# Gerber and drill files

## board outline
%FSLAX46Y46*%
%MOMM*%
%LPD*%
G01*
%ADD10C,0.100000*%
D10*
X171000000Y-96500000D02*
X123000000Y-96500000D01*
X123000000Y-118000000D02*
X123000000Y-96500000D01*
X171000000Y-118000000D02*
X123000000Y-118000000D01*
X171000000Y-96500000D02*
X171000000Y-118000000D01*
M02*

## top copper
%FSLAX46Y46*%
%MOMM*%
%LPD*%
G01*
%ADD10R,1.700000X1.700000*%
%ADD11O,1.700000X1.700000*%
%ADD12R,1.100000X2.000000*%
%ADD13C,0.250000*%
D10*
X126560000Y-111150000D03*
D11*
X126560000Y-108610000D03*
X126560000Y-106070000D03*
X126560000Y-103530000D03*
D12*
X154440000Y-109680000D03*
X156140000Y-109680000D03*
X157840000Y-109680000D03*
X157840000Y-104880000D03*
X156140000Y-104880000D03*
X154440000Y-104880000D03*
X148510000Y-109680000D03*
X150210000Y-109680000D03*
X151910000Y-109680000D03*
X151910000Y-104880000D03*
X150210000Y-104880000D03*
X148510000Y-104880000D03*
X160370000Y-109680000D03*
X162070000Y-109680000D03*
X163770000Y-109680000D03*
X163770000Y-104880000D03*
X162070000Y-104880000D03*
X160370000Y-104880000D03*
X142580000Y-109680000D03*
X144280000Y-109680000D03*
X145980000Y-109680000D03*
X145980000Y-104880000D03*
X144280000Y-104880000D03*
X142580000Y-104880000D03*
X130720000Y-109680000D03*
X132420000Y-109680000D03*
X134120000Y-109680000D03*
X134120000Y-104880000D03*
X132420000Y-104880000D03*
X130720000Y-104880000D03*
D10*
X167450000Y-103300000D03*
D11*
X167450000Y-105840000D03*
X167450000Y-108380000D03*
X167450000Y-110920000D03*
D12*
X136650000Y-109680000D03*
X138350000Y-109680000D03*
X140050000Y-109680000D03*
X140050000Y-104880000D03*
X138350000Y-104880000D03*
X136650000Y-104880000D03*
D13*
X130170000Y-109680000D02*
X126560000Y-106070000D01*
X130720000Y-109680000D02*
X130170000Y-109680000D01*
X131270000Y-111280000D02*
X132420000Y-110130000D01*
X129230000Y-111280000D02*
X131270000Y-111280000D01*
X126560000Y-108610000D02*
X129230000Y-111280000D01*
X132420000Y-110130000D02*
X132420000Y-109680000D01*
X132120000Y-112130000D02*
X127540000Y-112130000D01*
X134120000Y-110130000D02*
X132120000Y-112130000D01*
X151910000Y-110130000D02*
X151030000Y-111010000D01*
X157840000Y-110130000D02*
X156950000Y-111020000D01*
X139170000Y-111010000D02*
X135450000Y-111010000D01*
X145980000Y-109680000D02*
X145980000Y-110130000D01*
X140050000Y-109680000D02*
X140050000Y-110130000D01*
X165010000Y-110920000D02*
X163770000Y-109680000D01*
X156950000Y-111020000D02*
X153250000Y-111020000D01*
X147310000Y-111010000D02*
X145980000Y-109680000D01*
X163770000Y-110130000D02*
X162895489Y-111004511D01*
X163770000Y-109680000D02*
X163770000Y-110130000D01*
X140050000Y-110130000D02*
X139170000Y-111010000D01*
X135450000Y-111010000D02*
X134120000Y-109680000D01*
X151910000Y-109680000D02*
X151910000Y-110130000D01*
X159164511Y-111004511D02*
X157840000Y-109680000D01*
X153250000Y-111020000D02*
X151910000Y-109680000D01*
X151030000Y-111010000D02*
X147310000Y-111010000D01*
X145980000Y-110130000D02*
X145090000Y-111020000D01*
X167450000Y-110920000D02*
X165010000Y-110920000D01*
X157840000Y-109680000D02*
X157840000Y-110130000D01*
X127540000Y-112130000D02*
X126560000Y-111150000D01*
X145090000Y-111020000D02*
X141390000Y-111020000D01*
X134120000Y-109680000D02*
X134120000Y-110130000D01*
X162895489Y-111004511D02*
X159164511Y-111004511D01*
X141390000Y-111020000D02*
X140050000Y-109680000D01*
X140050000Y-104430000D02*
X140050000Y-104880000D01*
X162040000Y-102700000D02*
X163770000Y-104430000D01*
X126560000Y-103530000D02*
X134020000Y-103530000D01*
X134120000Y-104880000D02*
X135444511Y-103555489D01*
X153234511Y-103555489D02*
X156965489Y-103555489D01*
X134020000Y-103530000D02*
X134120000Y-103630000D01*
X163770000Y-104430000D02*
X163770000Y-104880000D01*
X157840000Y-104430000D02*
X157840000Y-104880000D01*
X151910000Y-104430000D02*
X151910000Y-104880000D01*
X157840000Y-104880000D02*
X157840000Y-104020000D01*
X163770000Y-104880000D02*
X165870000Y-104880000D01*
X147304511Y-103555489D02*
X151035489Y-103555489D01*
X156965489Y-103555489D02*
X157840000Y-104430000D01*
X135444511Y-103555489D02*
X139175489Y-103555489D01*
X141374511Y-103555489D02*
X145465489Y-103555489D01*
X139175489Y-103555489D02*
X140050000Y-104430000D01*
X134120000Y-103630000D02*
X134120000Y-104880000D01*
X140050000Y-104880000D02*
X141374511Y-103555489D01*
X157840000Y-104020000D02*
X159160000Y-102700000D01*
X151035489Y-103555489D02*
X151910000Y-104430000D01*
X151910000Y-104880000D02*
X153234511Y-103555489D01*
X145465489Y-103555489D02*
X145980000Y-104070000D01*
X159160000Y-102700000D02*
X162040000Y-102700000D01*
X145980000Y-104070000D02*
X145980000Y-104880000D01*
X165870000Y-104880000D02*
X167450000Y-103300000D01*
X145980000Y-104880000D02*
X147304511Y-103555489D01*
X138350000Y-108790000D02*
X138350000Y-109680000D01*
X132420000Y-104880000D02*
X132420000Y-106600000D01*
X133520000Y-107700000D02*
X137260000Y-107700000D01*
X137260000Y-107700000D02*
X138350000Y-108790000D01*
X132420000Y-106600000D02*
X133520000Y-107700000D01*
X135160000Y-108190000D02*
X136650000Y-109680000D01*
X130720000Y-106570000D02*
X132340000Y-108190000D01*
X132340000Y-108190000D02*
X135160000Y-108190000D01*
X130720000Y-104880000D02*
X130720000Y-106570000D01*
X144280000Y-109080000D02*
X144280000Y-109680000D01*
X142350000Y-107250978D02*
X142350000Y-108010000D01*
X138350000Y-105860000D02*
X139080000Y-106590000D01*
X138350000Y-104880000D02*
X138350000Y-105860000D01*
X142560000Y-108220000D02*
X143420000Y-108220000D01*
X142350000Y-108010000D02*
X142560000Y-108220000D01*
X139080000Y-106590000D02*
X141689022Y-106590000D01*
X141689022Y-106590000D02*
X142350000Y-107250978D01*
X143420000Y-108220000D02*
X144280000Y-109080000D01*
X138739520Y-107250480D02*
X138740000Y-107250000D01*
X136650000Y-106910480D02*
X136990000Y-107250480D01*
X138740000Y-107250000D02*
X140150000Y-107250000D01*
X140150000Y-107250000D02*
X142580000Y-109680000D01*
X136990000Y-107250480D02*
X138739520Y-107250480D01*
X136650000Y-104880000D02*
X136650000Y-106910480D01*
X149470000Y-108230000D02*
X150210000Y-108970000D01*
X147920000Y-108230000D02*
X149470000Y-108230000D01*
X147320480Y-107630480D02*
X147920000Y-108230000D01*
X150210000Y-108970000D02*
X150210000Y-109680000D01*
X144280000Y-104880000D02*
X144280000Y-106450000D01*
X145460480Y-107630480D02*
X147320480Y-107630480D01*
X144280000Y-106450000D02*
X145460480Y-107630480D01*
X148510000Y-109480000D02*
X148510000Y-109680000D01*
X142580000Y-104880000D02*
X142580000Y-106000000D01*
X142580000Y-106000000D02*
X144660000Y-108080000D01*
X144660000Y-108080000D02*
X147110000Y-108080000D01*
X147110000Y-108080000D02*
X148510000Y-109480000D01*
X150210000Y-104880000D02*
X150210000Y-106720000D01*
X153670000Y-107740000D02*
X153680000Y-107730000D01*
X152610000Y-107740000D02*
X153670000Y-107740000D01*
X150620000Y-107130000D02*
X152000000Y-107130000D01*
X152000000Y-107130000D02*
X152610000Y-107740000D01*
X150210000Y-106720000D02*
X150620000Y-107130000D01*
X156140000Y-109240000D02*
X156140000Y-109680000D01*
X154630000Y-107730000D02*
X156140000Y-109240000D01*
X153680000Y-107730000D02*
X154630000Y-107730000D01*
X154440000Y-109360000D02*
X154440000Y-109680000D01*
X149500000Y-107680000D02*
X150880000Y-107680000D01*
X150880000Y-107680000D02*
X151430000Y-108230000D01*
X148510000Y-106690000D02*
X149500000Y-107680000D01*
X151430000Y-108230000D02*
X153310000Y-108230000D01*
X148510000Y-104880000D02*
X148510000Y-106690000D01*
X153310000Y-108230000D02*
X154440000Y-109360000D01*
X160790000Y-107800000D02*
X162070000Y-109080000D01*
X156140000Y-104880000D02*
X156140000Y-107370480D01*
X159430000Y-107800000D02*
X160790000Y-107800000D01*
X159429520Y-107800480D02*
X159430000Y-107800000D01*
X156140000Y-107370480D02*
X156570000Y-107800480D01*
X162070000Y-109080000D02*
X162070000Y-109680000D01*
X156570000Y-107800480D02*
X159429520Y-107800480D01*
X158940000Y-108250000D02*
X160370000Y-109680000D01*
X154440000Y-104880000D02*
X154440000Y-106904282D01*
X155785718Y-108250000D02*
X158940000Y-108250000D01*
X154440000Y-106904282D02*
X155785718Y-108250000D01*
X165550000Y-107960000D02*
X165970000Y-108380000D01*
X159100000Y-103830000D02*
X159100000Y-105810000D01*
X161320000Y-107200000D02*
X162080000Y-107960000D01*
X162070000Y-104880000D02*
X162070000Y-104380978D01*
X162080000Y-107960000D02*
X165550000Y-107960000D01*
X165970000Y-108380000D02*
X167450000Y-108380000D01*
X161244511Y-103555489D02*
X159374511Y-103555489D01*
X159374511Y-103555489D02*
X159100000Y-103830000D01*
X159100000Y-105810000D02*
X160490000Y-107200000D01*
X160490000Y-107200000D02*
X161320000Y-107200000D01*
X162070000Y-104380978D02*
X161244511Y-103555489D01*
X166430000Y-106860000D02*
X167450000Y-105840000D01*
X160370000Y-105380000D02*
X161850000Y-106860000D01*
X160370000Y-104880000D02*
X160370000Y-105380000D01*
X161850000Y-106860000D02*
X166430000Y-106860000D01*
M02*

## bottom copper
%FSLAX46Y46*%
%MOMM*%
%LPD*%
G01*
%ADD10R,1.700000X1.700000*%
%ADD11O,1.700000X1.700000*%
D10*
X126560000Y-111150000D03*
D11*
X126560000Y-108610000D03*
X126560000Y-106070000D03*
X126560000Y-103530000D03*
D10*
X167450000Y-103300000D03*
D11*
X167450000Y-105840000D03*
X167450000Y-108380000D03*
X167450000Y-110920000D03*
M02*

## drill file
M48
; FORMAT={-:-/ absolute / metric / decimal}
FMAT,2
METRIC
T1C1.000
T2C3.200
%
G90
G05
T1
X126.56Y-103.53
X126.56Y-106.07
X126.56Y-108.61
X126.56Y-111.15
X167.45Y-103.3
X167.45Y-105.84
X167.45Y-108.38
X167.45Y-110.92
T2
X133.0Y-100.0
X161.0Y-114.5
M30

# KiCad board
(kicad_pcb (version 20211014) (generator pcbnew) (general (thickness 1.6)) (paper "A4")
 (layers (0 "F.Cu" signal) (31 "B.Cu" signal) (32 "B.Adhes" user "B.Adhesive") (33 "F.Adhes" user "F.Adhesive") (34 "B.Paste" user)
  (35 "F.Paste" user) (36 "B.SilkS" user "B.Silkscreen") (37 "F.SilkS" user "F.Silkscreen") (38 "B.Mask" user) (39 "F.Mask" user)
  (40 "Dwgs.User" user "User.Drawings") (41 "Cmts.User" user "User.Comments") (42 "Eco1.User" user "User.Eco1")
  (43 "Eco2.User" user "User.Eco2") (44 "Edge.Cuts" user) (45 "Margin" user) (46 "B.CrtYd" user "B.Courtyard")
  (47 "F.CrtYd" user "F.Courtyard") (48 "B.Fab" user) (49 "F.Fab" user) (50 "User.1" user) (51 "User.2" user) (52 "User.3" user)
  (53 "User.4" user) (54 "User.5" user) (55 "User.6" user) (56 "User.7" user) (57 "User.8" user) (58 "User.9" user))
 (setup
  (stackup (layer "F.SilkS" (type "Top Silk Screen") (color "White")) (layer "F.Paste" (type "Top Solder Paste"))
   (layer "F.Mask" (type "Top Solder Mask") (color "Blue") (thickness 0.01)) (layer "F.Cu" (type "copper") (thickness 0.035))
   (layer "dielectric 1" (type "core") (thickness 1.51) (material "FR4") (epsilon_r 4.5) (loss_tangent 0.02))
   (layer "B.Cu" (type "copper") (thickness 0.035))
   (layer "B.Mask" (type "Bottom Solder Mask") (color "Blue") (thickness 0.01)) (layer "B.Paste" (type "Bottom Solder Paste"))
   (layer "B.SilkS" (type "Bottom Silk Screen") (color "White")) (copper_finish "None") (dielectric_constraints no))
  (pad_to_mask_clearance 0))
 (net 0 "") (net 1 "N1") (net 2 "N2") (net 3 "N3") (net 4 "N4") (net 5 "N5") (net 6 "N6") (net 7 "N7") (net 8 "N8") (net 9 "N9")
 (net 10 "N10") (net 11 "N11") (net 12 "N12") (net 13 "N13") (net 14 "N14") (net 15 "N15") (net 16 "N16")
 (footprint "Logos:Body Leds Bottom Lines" (layer "F.Cu") (at 145.53 114.09)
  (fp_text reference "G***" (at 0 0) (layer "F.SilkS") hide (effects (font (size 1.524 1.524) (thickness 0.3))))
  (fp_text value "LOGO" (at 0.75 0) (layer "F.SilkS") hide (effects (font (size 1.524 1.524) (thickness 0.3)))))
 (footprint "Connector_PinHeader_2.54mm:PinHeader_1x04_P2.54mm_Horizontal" (layer "F.Cu") (at 126.56 111.15 180)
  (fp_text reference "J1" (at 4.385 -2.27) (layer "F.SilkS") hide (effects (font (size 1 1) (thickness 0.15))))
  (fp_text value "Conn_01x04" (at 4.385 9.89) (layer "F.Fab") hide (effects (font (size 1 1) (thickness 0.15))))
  (pad "1" thru_hole rect locked (at 0 0 180) (size 1.7 1.7) (drill 1) (layers *.Cu *.Mask) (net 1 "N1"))
  (pad "2" thru_hole oval locked (at 0 2.54 180) (size 1.7 1.7) (drill 1) (layers *.Cu *.Mask) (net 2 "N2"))
  (pad "3" thru_hole oval locked (at 0 5.08 180) (size 1.7 1.7) (drill 1) (layers *.Cu *.Mask) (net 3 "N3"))
  (pad "4" thru_hole oval locked (at 0 7.62 180) (size 1.7 1.7) (drill 1) (layers *.Cu *.Mask) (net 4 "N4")))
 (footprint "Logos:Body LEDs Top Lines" (layer "F.Cu") (at 151.18 101.11)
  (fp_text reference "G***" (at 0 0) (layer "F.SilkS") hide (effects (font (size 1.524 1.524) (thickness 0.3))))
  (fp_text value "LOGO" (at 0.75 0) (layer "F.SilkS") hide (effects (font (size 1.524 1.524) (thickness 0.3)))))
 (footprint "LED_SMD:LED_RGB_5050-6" (layer "F.Cu") (at 156.14 107.28 90)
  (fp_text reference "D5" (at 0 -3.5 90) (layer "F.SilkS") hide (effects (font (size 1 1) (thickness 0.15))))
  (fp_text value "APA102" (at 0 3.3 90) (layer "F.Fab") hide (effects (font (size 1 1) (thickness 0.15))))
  (pad "1" smd rect locked (at -2.4 -1.7 180) (size 1.1 2) (layers "F.Cu" "F.Paste" "F.Mask") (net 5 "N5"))
  (pad "2" smd rect locked (at -2.4 0 180) (size 1.1 2) (layers "F.Cu" "F.Paste" "F.Mask") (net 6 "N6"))
  (pad "3" smd rect locked (at -2.4 1.7 180) (size 1.1 2) (layers "F.Cu" "F.Paste" "F.Mask") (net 1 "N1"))
  (pad "4" smd rect locked (at 2.4 1.7 180) (size 1.1 2) (layers "F.Cu" "F.Paste" "F.Mask") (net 4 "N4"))
  (pad "5" smd rect locked (at 2.4 0 180) (size 1.1 2) (layers "F.Cu" "F.Paste" "F.Mask") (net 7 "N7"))
  (pad "6" smd rect locked (at 2.4 -1.7 180) (size 1.1 2) (layers "F.Cu" "F.Paste" "F.Mask") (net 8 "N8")))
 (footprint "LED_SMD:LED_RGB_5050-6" (layer "F.Cu") (at 150.21 107.28 90)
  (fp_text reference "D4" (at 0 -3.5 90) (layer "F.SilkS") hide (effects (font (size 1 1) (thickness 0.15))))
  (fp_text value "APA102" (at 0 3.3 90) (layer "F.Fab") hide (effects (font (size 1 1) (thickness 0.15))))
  (pad "1" smd rect locked (at -2.4 -1.7 180) (size 1.1 2) (layers "F.Cu" "F.Paste" "F.Mask") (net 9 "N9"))
  (pad "2" smd rect locked (at -2.4 0 180) (size 1.1 2) (layers "F.Cu" "F.Paste" "F.Mask") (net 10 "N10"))
  (pad "3" smd rect locked (at -2.4 1.7 180) (size 1.1 2) (layers "F.Cu" "F.Paste" "F.Mask") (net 1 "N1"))
  (pad "4" smd rect locked (at 2.4 1.7 180) (size 1.1 2) (layers "F.Cu" "F.Paste" "F.Mask") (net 4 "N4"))
  (pad "5" smd rect locked (at 2.4 0 180) (size 1.1 2) (layers "F.Cu" "F.Paste" "F.Mask") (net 6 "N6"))
  (pad "6" smd rect locked (at 2.4 -1.7 180) (size 1.1 2) (layers "F.Cu" "F.Paste" "F.Mask") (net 5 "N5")))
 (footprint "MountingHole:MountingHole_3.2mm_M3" (layer "F.Cu") (at 161 114.5)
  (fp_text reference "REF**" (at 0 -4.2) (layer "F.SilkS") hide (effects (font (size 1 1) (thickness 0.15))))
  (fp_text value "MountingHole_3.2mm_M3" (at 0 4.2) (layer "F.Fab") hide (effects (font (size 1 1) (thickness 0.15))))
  (pad "" np_thru_hole circle locked (at 0 0) (size 3.2 3.2) (drill 3.2) (layers *.Cu *.Mask)))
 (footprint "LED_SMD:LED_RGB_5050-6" (layer "F.Cu") (at 162.07 107.28 90)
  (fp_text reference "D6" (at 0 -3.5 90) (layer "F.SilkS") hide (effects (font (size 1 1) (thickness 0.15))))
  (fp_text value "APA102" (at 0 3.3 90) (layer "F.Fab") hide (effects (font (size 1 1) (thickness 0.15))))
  (pad "1" smd rect locked (at -2.4 -1.7 180) (size 1.1 2) (layers "F.Cu" "F.Paste" "F.Mask") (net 8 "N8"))
  (pad "2" smd rect locked (at -2.4 0 180) (size 1.1 2) (layers "F.Cu" "F.Paste" "F.Mask") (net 7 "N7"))
  (pad "3" smd rect locked (at -2.4 1.7 180) (size 1.1 2) (layers "F.Cu" "F.Paste" "F.Mask") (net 1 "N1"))
  (pad "4" smd rect locked (at 2.4 1.7 180) (size 1.1 2) (layers "F.Cu" "F.Paste" "F.Mask") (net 4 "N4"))
  (pad "5" smd rect locked (at 2.4 0 180) (size 1.1 2) (layers "F.Cu" "F.Paste" "F.Mask") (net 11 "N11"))
  (pad "6" smd rect locked (at 2.4 -1.7 180) (size 1.1 2) (layers "F.Cu" "F.Paste" "F.Mask") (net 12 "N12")))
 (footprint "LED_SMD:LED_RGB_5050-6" (layer "F.Cu") (at 144.28 107.28 90)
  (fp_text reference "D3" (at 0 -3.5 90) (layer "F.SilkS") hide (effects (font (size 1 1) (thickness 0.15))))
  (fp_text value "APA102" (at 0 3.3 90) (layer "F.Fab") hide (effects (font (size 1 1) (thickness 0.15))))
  (pad "1" smd rect locked (at -2.4 -1.7 180) (size 1.1 2) (layers "F.Cu" "F.Paste" "F.Mask") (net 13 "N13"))
  (pad "2" smd rect locked (at -2.4 0 180) (size 1.1 2) (layers "F.Cu" "F.Paste" "F.Mask") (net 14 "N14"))
  (pad "3" smd rect locked (at -2.4 1.7 180) (size 1.1 2) (layers "F.Cu" "F.Paste" "F.Mask") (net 1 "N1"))
  (pad "4" smd rect locked (at 2.4 1.7 180) (size 1.1 2) (layers "F.Cu" "F.Paste" "F.Mask") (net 4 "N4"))
  (pad "5" smd rect locked (at 2.4 0 180) (size 1.1 2) (layers "F.Cu" "F.Paste" "F.Mask") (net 10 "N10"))
  (pad "6" smd rect locked (at 2.4 -1.7 180) (size 1.1 2) (layers "F.Cu" "F.Paste" "F.Mask") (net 9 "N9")))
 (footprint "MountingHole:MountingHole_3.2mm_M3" (layer "F.Cu") (at 133 100)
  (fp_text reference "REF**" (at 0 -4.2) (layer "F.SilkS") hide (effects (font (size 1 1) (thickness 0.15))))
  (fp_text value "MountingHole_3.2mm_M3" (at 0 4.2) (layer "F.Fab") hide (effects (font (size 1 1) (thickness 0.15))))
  (pad "" np_thru_hole circle locked (at 0 0) (size 3.2 3.2) (drill 3.2) (layers *.Cu *.Mask)))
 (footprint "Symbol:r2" (layer "F.Cu") (at 130.49 114.52)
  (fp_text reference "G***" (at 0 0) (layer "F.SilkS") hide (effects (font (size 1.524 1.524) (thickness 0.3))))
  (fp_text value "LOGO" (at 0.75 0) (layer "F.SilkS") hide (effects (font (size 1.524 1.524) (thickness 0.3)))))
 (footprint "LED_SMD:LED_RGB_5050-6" (layer "F.Cu") (at 132.42 107.28 90)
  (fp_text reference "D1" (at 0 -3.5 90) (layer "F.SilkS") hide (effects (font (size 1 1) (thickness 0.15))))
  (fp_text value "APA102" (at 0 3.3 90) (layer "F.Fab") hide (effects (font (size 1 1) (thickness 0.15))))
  (pad "1" smd rect locked (at -2.4 -1.7 180) (size 1.1 2) (layers "F.Cu" "F.Paste" "F.Mask") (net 3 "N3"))
  (pad "2" smd rect locked (at -2.4 0 180) (size 1.1 2) (layers "F.Cu" "F.Paste" "F.Mask") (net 2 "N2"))
  (pad "3" smd rect locked (at -2.4 1.7 180) (size 1.1 2) (layers "F.Cu" "F.Paste" "F.Mask") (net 1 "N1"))
  (pad "4" smd rect locked (at 2.4 1.7 180) (size 1.1 2) (layers "F.Cu" "F.Paste" "F.Mask") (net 4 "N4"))
  (pad "5" smd rect locked (at 2.4 0 180) (size 1.1 2) (layers "F.Cu" "F.Paste" "F.Mask") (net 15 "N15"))
  (pad "6" smd rect locked (at 2.4 -1.7 180) (size 1.1 2) (layers "F.Cu" "F.Paste" "F.Mask") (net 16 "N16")))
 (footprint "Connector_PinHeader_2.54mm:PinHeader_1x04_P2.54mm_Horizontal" (layer "F.Cu") (at 167.45 103.3)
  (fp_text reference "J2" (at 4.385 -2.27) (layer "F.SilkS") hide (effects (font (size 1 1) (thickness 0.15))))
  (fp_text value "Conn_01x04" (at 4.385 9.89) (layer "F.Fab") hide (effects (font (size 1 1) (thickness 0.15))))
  (pad "1" thru_hole rect locked (at 0 0) (size 1.7 1.7) (drill 1) (layers *.Cu *.Mask) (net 4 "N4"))
  (pad "2" thru_hole oval locked (at 0 2.54) (size 1.7 1.7) (drill 1) (layers *.Cu *.Mask) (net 12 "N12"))
  (pad "3" thru_hole oval locked (at 0 5.08) (size 1.7 1.7) (drill 1) (layers *.Cu *.Mask) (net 11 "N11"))
  (pad "4" thru_hole oval locked (at 0 7.62) (size 1.7 1.7) (drill 1) (layers *.Cu *.Mask) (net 1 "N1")))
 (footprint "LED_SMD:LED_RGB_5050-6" (layer "F.Cu") (at 138.35 107.28 90)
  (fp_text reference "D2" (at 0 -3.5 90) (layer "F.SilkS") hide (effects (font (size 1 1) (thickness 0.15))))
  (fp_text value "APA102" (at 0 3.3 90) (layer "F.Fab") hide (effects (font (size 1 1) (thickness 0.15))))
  (pad "1" smd rect locked (at -2.4 -1.7 180) (size 1.1 2) (layers "F.Cu" "F.Paste" "F.Mask") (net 16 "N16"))
  (pad "2" smd rect locked (at -2.4 0 180) (size 1.1 2) (layers "F.Cu" "F.Paste" "F.Mask") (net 15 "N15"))
  (pad "3" smd rect locked (at -2.4 1.7 180) (size 1.1 2) (layers "F.Cu" "F.Paste" "F.Mask") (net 1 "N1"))
  (pad "4" smd rect locked (at 2.4 1.7 180) (size 1.1 2) (layers "F.Cu" "F.Paste" "F.Mask") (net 4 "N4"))
  (pad "5" smd rect locked (at 2.4 0 180) (size 1.1 2) (layers "F.Cu" "F.Paste" "F.Mask") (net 14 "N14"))
  (pad "6" smd rect locked (at 2.4 -1.7 180) (size 1.1 2) (layers "F.Cu" "F.Paste" "F.Mask") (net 13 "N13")))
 (gr_line (start 171 96.5) (end 123 96.5) (layer "Edge.Cuts") (width 0.1))
 (gr_line (start 123 118) (end 123 96.5) (layer "Edge.Cuts") (width 0.1))
 (gr_line (start 171 118) (end 123 118) (layer "Edge.Cuts") (width 0.1))
 (gr_line (start 171 96.5) (end 171 118) (layer "Edge.Cuts") (width 0.1))
 (segment (start 130.17 109.68) (end 126.56 106.07) (width 0.25) (layer "F.Cu") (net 3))
 (segment (start 130.72 109.68) (end 130.17 109.68) (width 0.25) (layer "F.Cu") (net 3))
 (segment (start 131.27 111.28) (end 132.42 110.13) (width 0.25) (layer "F.Cu") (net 2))
 (segment (start 129.23 111.28) (end 131.27 111.28) (width 0.25) (layer "F.Cu") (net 2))
 (segment (start 126.56 108.61) (end 129.23 111.28) (width 0.25) (layer "F.Cu") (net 2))
 (segment (start 132.42 110.13) (end 132.42 109.68) (width 0.25) (layer "F.Cu") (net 2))
 (segment (start 132.12 112.13) (end 127.54 112.13) (width 0.25) (layer "F.Cu") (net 1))
 (segment (start 134.12 110.13) (end 132.12 112.13) (width 0.25) (layer "F.Cu") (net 1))
 (segment (start 151.91 110.13) (end 151.03 111.01) (width 0.25) (layer "F.Cu") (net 1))
 (segment (start 157.84 110.13) (end 156.95 111.02) (width 0.25) (layer "F.Cu") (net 1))
 (segment (start 139.17 111.01) (end 135.45 111.01) (width 0.25) (layer "F.Cu") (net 1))
 (segment (start 145.98 109.68) (end 145.98 110.13) (width 0.25) (layer "F.Cu") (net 1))
 (segment (start 140.05 109.68) (end 140.05 110.13) (width 0.25) (layer "F.Cu") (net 1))
 (segment (start 165.01 110.92) (end 163.77 109.68) (width 0.25) (layer "F.Cu") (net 1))
 (segment (start 156.95 111.02) (end 153.25 111.02) (width 0.25) (layer "F.Cu") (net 1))
 (segment (start 147.31 111.01) (end 145.98 109.68) (width 0.25) (layer "F.Cu") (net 1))
 (segment (start 163.77 110.13) (end 162.895489 111.004511) (width 0.25) (layer "F.Cu") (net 1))
 (segment (start 163.77 109.68) (end 163.77 110.13) (width 0.25) (layer "F.Cu") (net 1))
 (segment (start 140.05 110.13) (end 139.17 111.01) (width 0.25) (layer "F.Cu") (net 1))
 (segment (start 135.45 111.01) (end 134.12 109.68) (width 0.25) (layer "F.Cu") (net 1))
 (segment (start 151.91 109.68) (end 151.91 110.13) (width 0.25) (layer "F.Cu") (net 1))
 (segment (start 159.164511 111.004511) (end 157.84 109.68) (width 0.25) (layer "F.Cu") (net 1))
 (segment (start 153.25 111.02) (end 151.91 109.68) (width 0.25) (layer "F.Cu") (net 1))
 (segment (start 151.03 111.01) (end 147.31 111.01) (width 0.25) (layer "F.Cu") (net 1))
 (segment (start 145.98 110.13) (end 145.09 111.02) (width 0.25) (layer "F.Cu") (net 1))
 (segment (start 167.45 110.92) (end 165.01 110.92) (width 0.25) (layer "F.Cu") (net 1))
 (segment (start 157.84 109.68) (end 157.84 110.13) (width 0.25) (layer "F.Cu") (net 1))
 (segment (start 127.54 112.13) (end 126.56 111.15) (width 0.25) (layer "F.Cu") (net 1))
 (segment (start 145.09 111.02) (end 141.39 111.02) (width 0.25) (layer "F.Cu") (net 1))
 (segment (start 134.12 109.68) (end 134.12 110.13) (width 0.25) (layer "F.Cu") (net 1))
 (segment (start 162.895489 111.004511) (end 159.164511 111.004511) (width 0.25) (layer "F.Cu") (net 1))
 (segment (start 141.39 111.02) (end 140.05 109.68) (width 0.25) (layer "F.Cu") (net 1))
 (segment (start 140.05 104.43) (end 140.05 104.88) (width 0.25) (layer "F.Cu") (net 4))
 (segment (start 162.04 102.7) (end 163.77 104.43) (width 0.25) (layer "F.Cu") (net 4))
 (segment (start 126.56 103.53) (end 134.02 103.53) (width 0.25) (layer "F.Cu") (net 4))
 (segment (start 134.12 104.88) (end 135.444511 103.555489) (width 0.25) (layer "F.Cu") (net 4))
 (segment (start 153.234511 103.555489) (end 156.965489 103.555489) (width 0.25) (layer "F.Cu") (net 4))
 (segment (start 134.02 103.53) (end 134.12 103.63) (width 0.25) (layer "F.Cu") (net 4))
 (segment (start 163.77 104.43) (end 163.77 104.88) (width 0.25) (layer "F.Cu") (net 4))
 (segment (start 157.84 104.43) (end 157.84 104.88) (width 0.25) (layer "F.Cu") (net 4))
 (segment (start 151.91 104.43) (end 151.91 104.88) (width 0.25) (layer "F.Cu") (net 4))
 (segment (start 157.84 104.88) (end 157.84 104.02) (width 0.25) (layer "F.Cu") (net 4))
 (segment (start 163.77 104.88) (end 165.87 104.88) (width 0.25) (layer "F.Cu") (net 4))
 (segment (start 147.304511 103.555489) (end 151.035489 103.555489) (width 0.25) (layer "F.Cu") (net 4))
 (segment (start 156.965489 103.555489) (end 157.84 104.43) (width 0.25) (layer "F.Cu") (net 4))
 (segment (start 135.444511 103.555489) (end 139.175489 103.555489) (width 0.25) (layer "F.Cu") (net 4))
 (segment (start 141.374511 103.555489) (end 145.465489 103.555489) (width 0.25) (layer "F.Cu") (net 4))
 (segment (start 139.175489 103.555489) (end 140.05 104.43) (width 0.25) (layer "F.Cu") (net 4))
 (segment (start 134.12 103.63) (end 134.12 104.88) (width 0.25) (layer "F.Cu") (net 4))
 (segment (start 140.05 104.88) (end 141.374511 103.555489) (width 0.25) (layer "F.Cu") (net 4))
 (segment (start 157.84 104.02) (end 159.16 102.7) (width 0.25) (layer "F.Cu") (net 4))
 (segment (start 151.035489 103.555489) (end 151.91 104.43) (width 0.25) (layer "F.Cu") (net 4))
 (segment (start 151.91 104.88) (end 153.234511 103.555489) (width 0.25) (layer "F.Cu") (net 4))
 (segment (start 145.465489 103.555489) (end 145.98 104.07) (width 0.25) (layer "F.Cu") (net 4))
 (segment (start 159.16 102.7) (end 162.04 102.7) (width 0.25) (layer "F.Cu") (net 4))
 (segment (start 145.98 104.07) (end 145.98 104.88) (width 0.25) (layer "F.Cu") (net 4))
 (segment (start 165.87 104.88) (end 167.45 103.3) (width 0.25) (layer "F.Cu") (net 4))
 (segment (start 145.98 104.88) (end 147.304511 103.555489) (width 0.25) (layer "F.Cu") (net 4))
 (segment (start 138.35 108.79) (end 138.35 109.68) (width 0.25) (layer "F.Cu") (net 15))
 (segment (start 132.42 104.88) (end 132.42 106.6) (width 0.25) (layer "F.Cu") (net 15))
 (segment (start 133.52 107.7) (end 137.26 107.7) (width 0.25) (layer "F.Cu") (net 15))
 (segment (start 137.26 107.7) (end 138.35 108.79) (width 0.25) (layer "F.Cu") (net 15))
 (segment (start 132.42 106.6) (end 133.52 107.7) (width 0.25) (layer "F.Cu") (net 15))
 (segment (start 135.16 108.19) (end 136.65 109.68) (width 0.25) (layer "F.Cu") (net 16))
 (segment (start 130.72 106.57) (end 132.34 108.19) (width 0.25) (layer "F.Cu") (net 16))
 (segment (start 132.34 108.19) (end 135.16 108.19) (width 0.25) (layer "F.Cu") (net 16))
 (segment (start 130.72 104.88) (end 130.72 106.57) (width 0.25) (layer "F.Cu") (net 16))
 (segment (start 144.28 109.08) (end 144.28 109.68) (width 0.25) (layer "F.Cu") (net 14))
 (segment (start 142.35 107.250978) (end 142.35 108.01) (width 0.25) (layer "F.Cu") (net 14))
 (segment (start 138.35 105.86) (end 139.08 106.59) (width 0.25) (layer "F.Cu") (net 14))
 (segment (start 138.35 104.88) (end 138.35 105.86) (width 0.25) (layer "F.Cu") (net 14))
 (segment (start 142.56 108.22) (end 143.42 108.22) (width 0.25) (layer "F.Cu") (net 14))
 (segment (start 142.35 108.01) (end 142.56 108.22) (width 0.25) (layer "F.Cu") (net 14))
 (segment (start 139.08 106.59) (end 141.689022 106.59) (width 0.25) (layer "F.Cu") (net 14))
 (segment (start 141.689022 106.59) (end 142.35 107.250978) (width 0.25) (layer "F.Cu") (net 14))
 (segment (start 143.42 108.22) (end 144.28 109.08) (width 0.25) (layer "F.Cu") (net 14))
 (segment (start 138.73952 107.25048) (end 138.74 107.25) (width 0.25) (layer "F.Cu") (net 13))
 (segment (start 136.65 106.91048) (end 136.99 107.25048) (width 0.25) (layer "F.Cu") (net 13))
 (segment (start 138.74 107.25) (end 140.15 107.25) (width 0.25) (layer "F.Cu") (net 13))
 (segment (start 140.15 107.25) (end 142.58 109.68) (width 0.25) (layer "F.Cu") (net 13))
 (segment (start 136.99 107.25048) (end 138.73952 107.25048) (width 0.25) (layer "F.Cu") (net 13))
 (segment (start 136.65 104.88) (end 136.65 106.91048) (width 0.25) (layer "F.Cu") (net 13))
 (segment (start 149.47 108.23) (end 150.21 108.97) (width 0.25) (layer "F.Cu") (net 10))
 (segment (start 147.92 108.23) (end 149.47 108.23) (width 0.25) (layer "F.Cu") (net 10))
 (segment (start 147.32048 107.63048) (end 147.92 108.23) (width 0.25) (layer "F.Cu") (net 10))
 (segment (start 150.21 108.97) (end 150.21 109.68) (width 0.25) (layer "F.Cu") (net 10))
 (segment (start 144.28 104.88) (end 144.28 106.45) (width 0.25) (layer "F.Cu") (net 10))
 (segment (start 145.46048 107.63048) (end 147.32048 107.63048) (width 0.25) (layer "F.Cu") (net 10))
 (segment (start 144.28 106.45) (end 145.46048 107.63048) (width 0.25) (layer "F.Cu") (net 10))
 (segment (start 148.51 109.48) (end 148.51 109.68) (width 0.25) (layer "F.Cu") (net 9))
 (segment (start 142.58 104.88) (end 142.58 106) (width 0.25) (layer "F.Cu") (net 9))
 (segment (start 142.58 106) (end 144.66 108.08) (width 0.25) (layer "F.Cu") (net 9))
 (segment (start 144.66 108.08) (end 147.11 108.08) (width 0.25) (layer "F.Cu") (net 9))
 (segment (start 147.11 108.08) (end 148.51 109.48) (width 0.25) (layer "F.Cu") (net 9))
 (segment (start 150.21 104.88) (end 150.21 106.72) (width 0.25) (layer "F.Cu") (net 6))
 (segment (start 153.67 107.74) (end 153.68 107.73) (width 0.25) (layer "F.Cu") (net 6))
 (segment (start 152.61 107.74) (end 153.67 107.74) (width 0.25) (layer "F.Cu") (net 6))
 (segment (start 150.62 107.13) (end 152 107.13) (width 0.25) (layer "F.Cu") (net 6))
 (segment (start 152 107.13) (end 152.61 107.74) (width 0.25) (layer "F.Cu") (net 6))
 (segment (start 150.21 106.72) (end 150.62 107.13) (width 0.25) (layer "F.Cu") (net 6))
 (segment (start 156.14 109.24) (end 156.14 109.68) (width 0.25) (layer "F.Cu") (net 6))
 (segment (start 154.63 107.73) (end 156.14 109.24) (width 0.25) (layer "F.Cu") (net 6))
 (segment (start 153.68 107.73) (end 154.63 107.73) (width 0.25) (layer "F.Cu") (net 6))
 (segment (start 154.44 109.36) (end 154.44 109.68) (width 0.25) (layer "F.Cu") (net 5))
 (segment (start 149.5 107.68) (end 150.88 107.68) (width 0.25) (layer "F.Cu") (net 5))
 (segment (start 150.88 107.68) (end 151.43 108.23) (width 0.25) (layer "F.Cu") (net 5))
 (segment (start 148.51 106.69) (end 149.5 107.68) (width 0.25) (layer "F.Cu") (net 5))
 (segment (start 151.43 108.23) (end 153.31 108.23) (width 0.25) (layer "F.Cu") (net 5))
 (segment (start 148.51 104.88) (end 148.51 106.69) (width 0.25) (layer "F.Cu") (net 5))
 (segment (start 153.31 108.23) (end 154.44 109.36) (width 0.25) (layer "F.Cu") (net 5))
 (segment (start 160.79 107.8) (end 162.07 109.08) (width 0.25) (layer "F.Cu") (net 7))
 (segment (start 156.14 104.88) (end 156.14 107.37048) (width 0.25) (layer "F.Cu") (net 7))
 (segment (start 159.43 107.8) (end 160.79 107.8) (width 0.25) (layer "F.Cu") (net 7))
 (segment (start 159.42952 107.80048) (end 159.43 107.8) (width 0.25) (layer "F.Cu") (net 7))
 (segment (start 156.14 107.37048) (end 156.57 107.80048) (width 0.25) (layer "F.Cu") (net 7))
 (segment (start 162.07 109.08) (end 162.07 109.68) (width 0.25) (layer "F.Cu") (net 7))
 (segment (start 156.57 107.80048) (end 159.42952 107.80048) (width 0.25) (layer "F.Cu") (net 7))
 (segment (start 158.94 108.25) (end 160.37 109.68) (width 0.25) (layer "F.Cu") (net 8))
 (segment (start 154.44 104.88) (end 154.44 106.904282) (width 0.25) (layer "F.Cu") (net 8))
 (segment (start 155.785718 108.25) (end 158.94 108.25) (width 0.25) (layer "F.Cu") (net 8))
 (segment (start 154.44 106.904282) (end 155.785718 108.25) (width 0.25) (layer "F.Cu") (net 8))
 (segment (start 165.55 107.96) (end 165.97 108.38) (width 0.25) (layer "F.Cu") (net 11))
 (segment (start 159.1 103.83) (end 159.1 105.81) (width 0.25) (layer "F.Cu") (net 11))
 (segment (start 161.32 107.2) (end 162.08 107.96) (width 0.25) (layer "F.Cu") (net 11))
 (segment (start 162.07 104.88) (end 162.07 104.380978) (width 0.25) (layer "F.Cu") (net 11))
 (segment (start 162.08 107.96) (end 165.55 107.96) (width 0.25) (layer "F.Cu") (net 11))
 (segment (start 165.97 108.38) (end 167.45 108.38) (width 0.25) (layer "F.Cu") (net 11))
 (segment (start 161.244511 103.555489) (end 159.374511 103.555489) (width 0.25) (layer "F.Cu") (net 11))
 (segment (start 159.374511 103.555489) (end 159.1 103.83) (width 0.25) (layer "F.Cu") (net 11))
 (segment (start 159.1 105.81) (end 160.49 107.2) (width 0.25) (layer "F.Cu") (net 11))
 (segment (start 160.49 107.2) (end 161.32 107.2) (width 0.25) (layer "F.Cu") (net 11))
 (segment (start 162.07 104.380978) (end 161.244511 103.555489) (width 0.25) (layer "F.Cu") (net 11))
 (segment (start 166.43 106.86) (end 167.45 105.84) (width 0.25) (layer "F.Cu") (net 12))
 (segment (start 160.37 105.38) (end 161.85 106.86) (width 0.25) (layer "F.Cu") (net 12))
 (segment (start 160.37 104.88) (end 160.37 105.38) (width 0.25) (layer "F.Cu") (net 12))
 (segment (start 161.85 106.86) (end 166.43 106.86) (width 0.25) (layer "F.Cu") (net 12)))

